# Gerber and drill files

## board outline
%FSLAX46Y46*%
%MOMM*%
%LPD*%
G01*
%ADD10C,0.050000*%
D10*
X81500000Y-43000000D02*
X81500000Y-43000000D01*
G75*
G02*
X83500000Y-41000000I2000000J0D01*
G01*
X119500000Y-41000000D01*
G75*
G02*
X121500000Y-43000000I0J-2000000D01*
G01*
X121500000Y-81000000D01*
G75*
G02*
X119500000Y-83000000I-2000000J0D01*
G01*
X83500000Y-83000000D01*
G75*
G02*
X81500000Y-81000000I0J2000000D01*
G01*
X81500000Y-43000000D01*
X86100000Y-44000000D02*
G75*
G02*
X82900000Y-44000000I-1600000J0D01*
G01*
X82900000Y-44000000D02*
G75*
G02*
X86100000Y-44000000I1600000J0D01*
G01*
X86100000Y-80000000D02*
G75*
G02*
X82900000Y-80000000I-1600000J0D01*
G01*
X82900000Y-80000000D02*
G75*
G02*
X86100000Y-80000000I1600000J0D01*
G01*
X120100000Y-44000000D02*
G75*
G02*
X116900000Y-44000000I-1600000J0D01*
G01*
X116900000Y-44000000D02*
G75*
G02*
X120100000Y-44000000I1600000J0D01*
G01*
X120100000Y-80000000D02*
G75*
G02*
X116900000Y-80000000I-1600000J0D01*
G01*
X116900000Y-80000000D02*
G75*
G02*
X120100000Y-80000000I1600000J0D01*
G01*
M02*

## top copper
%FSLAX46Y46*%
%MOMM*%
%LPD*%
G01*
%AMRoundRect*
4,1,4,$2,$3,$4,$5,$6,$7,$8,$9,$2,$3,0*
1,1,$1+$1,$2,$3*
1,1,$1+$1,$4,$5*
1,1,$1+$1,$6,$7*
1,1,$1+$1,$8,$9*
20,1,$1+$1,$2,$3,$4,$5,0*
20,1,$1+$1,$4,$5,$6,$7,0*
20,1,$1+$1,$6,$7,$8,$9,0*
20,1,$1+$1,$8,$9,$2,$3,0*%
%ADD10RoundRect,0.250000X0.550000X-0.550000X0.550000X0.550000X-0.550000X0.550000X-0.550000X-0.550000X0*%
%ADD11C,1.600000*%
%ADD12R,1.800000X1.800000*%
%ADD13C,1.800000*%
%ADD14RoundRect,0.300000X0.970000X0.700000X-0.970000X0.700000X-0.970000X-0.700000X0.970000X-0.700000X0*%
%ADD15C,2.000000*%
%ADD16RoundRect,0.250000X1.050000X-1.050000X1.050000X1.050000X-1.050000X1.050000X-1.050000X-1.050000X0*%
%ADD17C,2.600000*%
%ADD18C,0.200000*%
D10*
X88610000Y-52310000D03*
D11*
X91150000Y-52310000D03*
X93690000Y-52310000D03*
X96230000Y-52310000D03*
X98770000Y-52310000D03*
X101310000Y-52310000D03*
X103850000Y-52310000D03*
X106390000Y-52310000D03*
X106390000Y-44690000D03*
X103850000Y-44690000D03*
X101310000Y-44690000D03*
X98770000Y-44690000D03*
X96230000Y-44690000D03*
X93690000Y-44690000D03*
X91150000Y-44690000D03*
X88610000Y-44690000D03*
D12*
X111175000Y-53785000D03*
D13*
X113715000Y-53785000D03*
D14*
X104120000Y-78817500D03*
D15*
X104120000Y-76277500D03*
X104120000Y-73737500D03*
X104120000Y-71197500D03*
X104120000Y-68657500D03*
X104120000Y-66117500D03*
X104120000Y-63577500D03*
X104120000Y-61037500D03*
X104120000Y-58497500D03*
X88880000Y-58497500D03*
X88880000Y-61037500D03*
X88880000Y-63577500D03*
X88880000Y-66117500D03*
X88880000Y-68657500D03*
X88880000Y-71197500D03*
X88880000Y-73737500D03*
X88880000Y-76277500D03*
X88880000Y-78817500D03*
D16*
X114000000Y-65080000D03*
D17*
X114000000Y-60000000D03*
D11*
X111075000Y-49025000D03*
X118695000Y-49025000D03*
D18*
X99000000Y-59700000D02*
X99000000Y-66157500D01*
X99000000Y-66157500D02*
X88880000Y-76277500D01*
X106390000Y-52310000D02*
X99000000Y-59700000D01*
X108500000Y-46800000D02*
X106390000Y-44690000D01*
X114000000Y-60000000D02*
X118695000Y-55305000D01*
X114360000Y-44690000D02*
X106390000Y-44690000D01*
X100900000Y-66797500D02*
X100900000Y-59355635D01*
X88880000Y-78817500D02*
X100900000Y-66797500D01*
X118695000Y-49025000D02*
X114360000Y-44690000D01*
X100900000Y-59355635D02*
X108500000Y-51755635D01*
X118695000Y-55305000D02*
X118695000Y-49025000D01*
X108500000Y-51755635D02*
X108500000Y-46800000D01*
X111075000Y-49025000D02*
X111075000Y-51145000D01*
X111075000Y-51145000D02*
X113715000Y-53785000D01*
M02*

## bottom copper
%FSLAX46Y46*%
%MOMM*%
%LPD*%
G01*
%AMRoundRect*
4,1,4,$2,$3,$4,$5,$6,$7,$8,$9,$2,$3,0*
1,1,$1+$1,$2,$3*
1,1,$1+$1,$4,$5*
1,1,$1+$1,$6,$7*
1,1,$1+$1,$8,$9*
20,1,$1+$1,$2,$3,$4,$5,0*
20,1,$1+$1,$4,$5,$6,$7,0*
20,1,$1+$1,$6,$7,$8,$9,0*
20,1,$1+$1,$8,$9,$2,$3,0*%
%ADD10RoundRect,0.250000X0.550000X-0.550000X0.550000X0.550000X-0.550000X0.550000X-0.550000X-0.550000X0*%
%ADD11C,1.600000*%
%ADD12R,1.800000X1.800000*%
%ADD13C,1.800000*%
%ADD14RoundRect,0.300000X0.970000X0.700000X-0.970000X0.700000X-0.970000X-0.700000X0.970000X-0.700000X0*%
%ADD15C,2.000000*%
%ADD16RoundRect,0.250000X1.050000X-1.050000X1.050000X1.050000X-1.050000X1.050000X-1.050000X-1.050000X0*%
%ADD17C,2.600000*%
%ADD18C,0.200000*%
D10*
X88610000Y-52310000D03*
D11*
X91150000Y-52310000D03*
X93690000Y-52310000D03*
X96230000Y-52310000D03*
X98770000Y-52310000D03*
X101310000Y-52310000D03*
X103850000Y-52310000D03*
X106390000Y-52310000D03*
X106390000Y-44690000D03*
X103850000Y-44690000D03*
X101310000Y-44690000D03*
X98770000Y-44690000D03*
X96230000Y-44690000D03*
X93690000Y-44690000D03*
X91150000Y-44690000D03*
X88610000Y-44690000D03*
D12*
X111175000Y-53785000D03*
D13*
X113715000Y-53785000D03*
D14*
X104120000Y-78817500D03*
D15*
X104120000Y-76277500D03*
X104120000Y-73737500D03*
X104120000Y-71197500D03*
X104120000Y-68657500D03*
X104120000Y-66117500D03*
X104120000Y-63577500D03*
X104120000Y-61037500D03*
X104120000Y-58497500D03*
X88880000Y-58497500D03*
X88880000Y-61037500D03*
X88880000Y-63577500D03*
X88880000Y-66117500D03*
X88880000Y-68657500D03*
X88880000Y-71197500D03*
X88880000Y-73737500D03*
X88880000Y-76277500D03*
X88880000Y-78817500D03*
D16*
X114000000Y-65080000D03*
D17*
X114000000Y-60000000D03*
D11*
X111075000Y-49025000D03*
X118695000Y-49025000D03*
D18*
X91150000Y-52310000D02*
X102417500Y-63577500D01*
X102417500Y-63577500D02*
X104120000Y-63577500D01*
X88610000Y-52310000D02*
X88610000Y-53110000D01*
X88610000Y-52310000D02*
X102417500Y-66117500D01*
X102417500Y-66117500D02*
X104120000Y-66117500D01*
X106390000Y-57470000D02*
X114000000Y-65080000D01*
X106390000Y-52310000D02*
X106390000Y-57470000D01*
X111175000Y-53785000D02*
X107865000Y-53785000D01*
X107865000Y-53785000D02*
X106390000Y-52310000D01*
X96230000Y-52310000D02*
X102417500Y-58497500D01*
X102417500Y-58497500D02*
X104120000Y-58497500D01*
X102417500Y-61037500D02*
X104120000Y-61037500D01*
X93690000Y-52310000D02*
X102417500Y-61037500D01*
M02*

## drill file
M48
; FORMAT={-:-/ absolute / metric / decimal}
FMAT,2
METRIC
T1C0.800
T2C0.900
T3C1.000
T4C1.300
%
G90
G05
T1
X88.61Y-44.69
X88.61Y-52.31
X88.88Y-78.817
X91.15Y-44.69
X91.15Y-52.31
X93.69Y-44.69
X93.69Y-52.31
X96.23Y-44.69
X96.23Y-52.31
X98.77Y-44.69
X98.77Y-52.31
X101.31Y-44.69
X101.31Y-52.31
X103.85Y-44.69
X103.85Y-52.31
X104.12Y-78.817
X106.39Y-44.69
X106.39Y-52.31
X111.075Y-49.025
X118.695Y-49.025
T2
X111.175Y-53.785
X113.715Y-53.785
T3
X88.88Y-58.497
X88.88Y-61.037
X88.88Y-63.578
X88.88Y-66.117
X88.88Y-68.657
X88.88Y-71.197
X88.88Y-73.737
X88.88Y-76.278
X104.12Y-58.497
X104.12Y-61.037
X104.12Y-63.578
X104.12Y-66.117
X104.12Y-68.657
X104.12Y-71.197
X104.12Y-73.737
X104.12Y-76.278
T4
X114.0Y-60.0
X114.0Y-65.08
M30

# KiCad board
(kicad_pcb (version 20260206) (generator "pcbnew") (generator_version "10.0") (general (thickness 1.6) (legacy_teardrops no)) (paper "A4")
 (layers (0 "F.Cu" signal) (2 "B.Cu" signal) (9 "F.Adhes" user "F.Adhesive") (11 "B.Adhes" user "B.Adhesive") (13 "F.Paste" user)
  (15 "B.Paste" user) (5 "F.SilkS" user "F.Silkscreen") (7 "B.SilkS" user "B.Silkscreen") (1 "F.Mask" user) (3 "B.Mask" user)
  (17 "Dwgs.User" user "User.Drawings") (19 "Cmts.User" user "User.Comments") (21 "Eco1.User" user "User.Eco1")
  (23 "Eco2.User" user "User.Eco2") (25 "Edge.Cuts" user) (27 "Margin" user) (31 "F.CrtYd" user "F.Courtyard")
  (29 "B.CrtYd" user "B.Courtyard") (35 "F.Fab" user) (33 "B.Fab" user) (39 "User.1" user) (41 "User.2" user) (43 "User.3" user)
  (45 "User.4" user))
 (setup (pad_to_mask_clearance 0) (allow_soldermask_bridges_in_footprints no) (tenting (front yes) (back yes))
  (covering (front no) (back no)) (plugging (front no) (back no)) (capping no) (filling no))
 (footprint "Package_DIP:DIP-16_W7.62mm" (layer "F.Cu") (at 88.61 52.31 90)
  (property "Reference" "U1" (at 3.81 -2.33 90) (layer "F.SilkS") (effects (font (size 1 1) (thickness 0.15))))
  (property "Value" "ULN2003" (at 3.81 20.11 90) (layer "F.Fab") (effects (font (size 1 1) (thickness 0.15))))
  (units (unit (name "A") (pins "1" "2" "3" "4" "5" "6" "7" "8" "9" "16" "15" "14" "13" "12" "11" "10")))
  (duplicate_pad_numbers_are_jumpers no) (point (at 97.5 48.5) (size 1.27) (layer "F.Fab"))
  (pad "1" thru_hole roundrect (at 0 0 90) (size 1.6 1.6) (drill 0.8) (layers "*.Cu" "*.Mask") (remove_unused_layers no)
   (roundrect_rratio 0.15625) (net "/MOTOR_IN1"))
  (pad "2" thru_hole circle (at 0 2.54 90) (size 1.6 1.6) (drill 0.8) (layers "*.Cu" "*.Mask") (remove_unused_layers no) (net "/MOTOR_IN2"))
  (pad "3" thru_hole circle (at 0 5.08 90) (size 1.6 1.6) (drill 0.8) (layers "*.Cu" "*.Mask") (remove_unused_layers no) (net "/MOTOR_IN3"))
  (pad "4" thru_hole circle (at 0 7.62 90) (size 1.6 1.6) (drill 0.8) (layers "*.Cu" "*.Mask") (remove_unused_layers no) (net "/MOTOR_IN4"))
  (pad "5" thru_hole circle (at 0 10.16 90) (size 1.6 1.6) (drill 0.8) (layers "*.Cu" "*.Mask") (remove_unused_layers no)
   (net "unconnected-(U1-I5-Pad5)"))
  (pad "6" thru_hole circle (at 0 12.7 90) (size 1.6 1.6) (drill 0.8) (layers "*.Cu" "*.Mask") (remove_unused_layers no)
   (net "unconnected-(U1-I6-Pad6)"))
  (pad "7" thru_hole circle (at 0 15.24 90) (size 1.6 1.6) (drill 0.8) (layers "*.Cu" "*.Mask") (remove_unused_layers no)
   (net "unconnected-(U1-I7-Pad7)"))
  (pad "8" thru_hole circle (at 0 17.78 90) (size 1.6 1.6) (drill 0.8) (layers "*.Cu" "*.Mask") (remove_unused_layers no) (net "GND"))
  (pad "9" thru_hole circle (at 7.62 17.78 90) (size 1.6 1.6) (drill 0.8) (layers "*.Cu" "*.Mask") (remove_unused_layers no) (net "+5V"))
  (pad "10" thru_hole circle (at 7.62 15.24 90) (size 1.6 1.6) (drill 0.8) (layers "*.Cu" "*.Mask") (remove_unused_layers no)
   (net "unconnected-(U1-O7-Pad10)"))
  (pad "11" thru_hole circle (at 7.62 12.7 90) (size 1.6 1.6) (drill 0.8) (layers "*.Cu" "*.Mask") (remove_unused_layers no)
   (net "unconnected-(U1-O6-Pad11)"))
  (pad "12" thru_hole circle (at 7.62 10.16 90) (size 1.6 1.6) (drill 0.8) (layers "*.Cu" "*.Mask") (remove_unused_layers no)
   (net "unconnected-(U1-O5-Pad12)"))
  (pad "13" thru_hole circle (at 7.62 7.62 90) (size 1.6 1.6) (drill 0.8) (layers "*.Cu" "*.Mask") (remove_unused_layers no)
   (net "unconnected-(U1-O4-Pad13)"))
  (pad "14" thru_hole circle (at 7.62 5.08 90) (size 1.6 1.6) (drill 0.8) (layers "*.Cu" "*.Mask") (remove_unused_layers no)
   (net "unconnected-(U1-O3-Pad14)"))
  (pad "15" thru_hole circle (at 7.62 2.54 90) (size 1.6 1.6) (drill 0.8) (layers "*.Cu" "*.Mask") (remove_unused_layers no)
   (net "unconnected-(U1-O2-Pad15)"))
  (pad "16" thru_hole circle (at 7.62 0 90) (size 1.6 1.6) (drill 0.8) (layers "*.Cu" "*.Mask") (remove_unused_layers no)
   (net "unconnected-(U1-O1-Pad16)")))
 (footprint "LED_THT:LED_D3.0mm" (layer "F.Cu") (at 111.175 53.785)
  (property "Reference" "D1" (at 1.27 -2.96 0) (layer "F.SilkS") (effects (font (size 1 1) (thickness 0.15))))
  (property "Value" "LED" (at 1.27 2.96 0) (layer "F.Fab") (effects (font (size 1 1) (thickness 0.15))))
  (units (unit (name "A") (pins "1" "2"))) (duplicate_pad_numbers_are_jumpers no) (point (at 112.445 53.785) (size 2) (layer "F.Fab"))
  (pad "1" thru_hole rect (at 0 0) (size 1.8 1.8) (drill 0.9) (layers "*.Cu" "*.Mask") (remove_unused_layers no) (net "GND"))
  (pad "2" thru_hole circle (at 2.54 0) (size 1.8 1.8) (drill 0.9) (layers "*.Cu" "*.Mask") (remove_unused_layers no) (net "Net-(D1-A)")))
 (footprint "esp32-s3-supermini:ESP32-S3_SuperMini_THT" (layer "F.Cu") (at 104.12 78.8175 180)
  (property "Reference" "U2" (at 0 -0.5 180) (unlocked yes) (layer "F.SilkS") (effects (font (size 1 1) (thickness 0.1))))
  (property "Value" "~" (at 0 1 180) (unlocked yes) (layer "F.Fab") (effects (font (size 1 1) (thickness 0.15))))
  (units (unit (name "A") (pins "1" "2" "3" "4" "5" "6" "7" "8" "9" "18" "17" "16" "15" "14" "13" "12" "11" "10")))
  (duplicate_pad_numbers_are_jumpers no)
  (pad "1" thru_hole roundrect (at 0 0 180) (size 2.54 2) (drill 0.8) (layers "*.Cu" "*.Mask") (remove_unused_layers no)
   (roundrect_rratio 0.15) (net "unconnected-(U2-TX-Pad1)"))
  (pad "2" thru_hole circle (at 0 2.54 180) (size 2 2) (drill 1) (layers "*.Cu" "*.Mask") (remove_unused_layers no)
   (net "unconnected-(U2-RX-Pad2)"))
  (pad "3" thru_hole circle (at 0 5.08 180) (size 2 2) (drill 1) (layers "*.Cu" "*.Mask") (remove_unused_layers no)
   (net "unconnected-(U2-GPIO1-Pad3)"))
  (pad "4" thru_hole circle (at 0 7.62 180) (size 2 2) (drill 1) (layers "*.Cu" "*.Mask") (remove_unused_layers no)
   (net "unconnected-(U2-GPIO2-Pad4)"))
  (pad "5" thru_hole circle (at 0 10.16 180) (size 2 2) (drill 1) (layers "*.Cu" "*.Mask") (remove_unused_layers no)
   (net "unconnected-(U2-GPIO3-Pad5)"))
  (pad "6" thru_hole circle (at 0 12.7 180) (size 2 2) (drill 1) (layers "*.Cu" "*.Mask") (remove_unused_layers no) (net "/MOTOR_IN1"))
  (pad "7" thru_hole circle (at 0 15.24 180) (size 2 2) (drill 1) (layers "*.Cu" "*.Mask") (remove_unused_layers no) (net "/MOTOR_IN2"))
  (pad "8" thru_hole circle (at 0 17.78 180) (size 2 2) (drill 1) (layers "*.Cu" "*.Mask") (remove_unused_layers no) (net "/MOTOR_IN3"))
  (pad "9" thru_hole circle (at 0 20.32 180) (size 2 2) (drill 1) (layers "*.Cu" "*.Mask") (remove_unused_layers no) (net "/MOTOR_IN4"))
  (pad "10" thru_hole circle (at 15.24 20.32 180) (size 2 2) (drill 1) (layers "*.Cu" "*.Mask") (remove_unused_layers no)
   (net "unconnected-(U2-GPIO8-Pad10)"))
  (pad "11" thru_hole circle (at 15.24 17.78 180) (size 2 2) (drill 1) (layers "*.Cu" "*.Mask") (remove_unused_layers no)
   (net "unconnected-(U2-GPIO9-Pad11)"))
  (pad "12" thru_hole circle (at 15.24 15.24 180) (size 2 2) (drill 1) (layers "*.Cu" "*.Mask") (remove_unused_layers no)
   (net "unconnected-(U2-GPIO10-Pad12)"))
  (pad "13" thru_hole circle (at 15.24 12.7 180) (size 2 2) (drill 1) (layers "*.Cu" "*.Mask") (remove_unused_layers no)
   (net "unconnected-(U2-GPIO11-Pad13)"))
  (pad "14" thru_hole circle (at 15.24 10.16 180) (size 2 2) (drill 1) (layers "*.Cu" "*.Mask") (remove_unused_layers no)
   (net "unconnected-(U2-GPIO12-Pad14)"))
  (pad "15" thru_hole circle (at 15.24 7.62 180) (size 2 2) (drill 1) (layers "*.Cu" "*.Mask") (remove_unused_layers no)
   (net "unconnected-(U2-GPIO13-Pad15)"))
  (pad "16" thru_hole circle (at 15.24 5.08 180) (size 2 2) (drill 1) (layers "*.Cu" "*.Mask") (remove_unused_layers no)
   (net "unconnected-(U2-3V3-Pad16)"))
  (pad "17" thru_hole circle (at 15.24 2.54 180) (size 2 2) (drill 1) (layers "*.Cu" "*.Mask") (remove_unused_layers no) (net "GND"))
  (pad "18" thru_hole circle (at 15.24 0 180) (size 2 2) (drill 0.8) (layers "*.Cu" "*.Mask") (remove_unused_layers no) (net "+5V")))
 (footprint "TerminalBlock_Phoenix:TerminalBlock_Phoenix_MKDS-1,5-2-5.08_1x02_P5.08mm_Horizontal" (layer "F.Cu") (at 114 65.08 90)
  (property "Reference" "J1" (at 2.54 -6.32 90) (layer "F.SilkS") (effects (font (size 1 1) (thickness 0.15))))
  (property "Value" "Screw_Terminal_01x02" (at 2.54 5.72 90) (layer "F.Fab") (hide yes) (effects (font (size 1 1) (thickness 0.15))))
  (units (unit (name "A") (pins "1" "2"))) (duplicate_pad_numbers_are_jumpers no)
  (pad "1" thru_hole roundrect (at 0 0 90) (size 2.6 2.6) (drill 1.3) (layers "*.Cu" "*.Mask") (remove_unused_layers no)
   (roundrect_rratio 0.096154) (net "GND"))
  (pad "2" thru_hole circle (at 5.08 0 90) (size 2.6 2.6) (drill 1.3) (layers "*.Cu" "*.Mask") (remove_unused_layers no) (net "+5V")))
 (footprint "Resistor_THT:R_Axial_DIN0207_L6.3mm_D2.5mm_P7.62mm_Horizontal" (layer "F.Cu") (at 111.075 49.025)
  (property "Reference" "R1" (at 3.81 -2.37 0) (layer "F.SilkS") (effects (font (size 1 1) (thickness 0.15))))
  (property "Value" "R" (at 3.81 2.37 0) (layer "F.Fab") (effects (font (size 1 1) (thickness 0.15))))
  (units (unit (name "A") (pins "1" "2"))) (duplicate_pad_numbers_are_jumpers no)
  (pad "1" thru_hole circle (at 0 0) (size 1.6 1.6) (drill 0.8) (layers "*.Cu" "*.Mask") (remove_unused_layers no) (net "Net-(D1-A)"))
  (pad "2" thru_hole circle (at 7.62 0) (size 1.6 1.6) (drill 0.8) (layers "*.Cu" "*.Mask") (remove_unused_layers no) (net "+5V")))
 (gr_rect (start 81.5 41) (end 121.5 83) (radius 2) (stroke (width 0.05) (type solid)) (fill no) (layer "Edge.Cuts"))
 (gr_circle (center 84.5 44) (end 86.1 44) (stroke (width 0.05) (type solid)) (fill no) (layer "Edge.Cuts"))
 (gr_circle (center 84.5 80) (end 86.1 80) (stroke (width 0.05) (type solid)) (fill no) (layer "Edge.Cuts"))
 (gr_circle (center 118.5 44) (end 120.1 44) (stroke (width 0.05) (type solid)) (fill no) (layer "Edge.Cuts"))
 (gr_circle (center 118.5 80) (end 120.1 80) (stroke (width 0.05) (type solid)) (fill no) (layer "Edge.Cuts"))
 (segment (start 91.15 52.31) (end 102.4175 63.5775) (width 0.2) (layer "B.Cu") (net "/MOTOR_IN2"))
 (segment (start 102.4175 63.5775) (end 104.12 63.5775) (width 0.2) (layer "B.Cu") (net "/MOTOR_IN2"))
 (segment (start 88.61 52.31) (end 88.61 53.11) (width 0.2) (layer "B.Cu") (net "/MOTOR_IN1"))
 (segment (start 88.61 52.31) (end 102.4175 66.1175) (width 0.2) (layer "B.Cu") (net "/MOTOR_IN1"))
 (segment (start 102.4175 66.1175) (end 104.12 66.1175) (width 0.2) (layer "B.Cu") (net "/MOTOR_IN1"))
 (segment (start 99 59.7) (end 99 66.1575) (width 0.2) (layer "F.Cu") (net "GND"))
 (segment (start 99 66.1575) (end 88.88 76.2775) (width 0.2) (layer "F.Cu") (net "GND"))
 (segment (start 106.39 52.31) (end 99 59.7) (width 0.2) (layer "F.Cu") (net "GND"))
 (segment (start 106.39 57.47) (end 114 65.08) (width 0.2) (layer "B.Cu") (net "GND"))
 (segment (start 106.39 52.31) (end 106.39 57.47) (width 0.2) (layer "B.Cu") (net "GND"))
 (segment (start 111.175 53.785) (end 107.865 53.785) (width 0.2) (layer "B.Cu") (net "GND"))
 (segment (start 107.865 53.785) (end 106.39 52.31) (width 0.2) (layer "B.Cu") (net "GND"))
 (segment (start 108.5 46.8) (end 106.39 44.69) (width 0.2) (layer "F.Cu") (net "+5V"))
 (segment (start 114 60) (end 118.695 55.305) (width 0.2) (layer "F.Cu") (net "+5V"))
 (segment (start 114.36 44.69) (end 106.39 44.69) (width 0.2) (layer "F.Cu") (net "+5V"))
 (segment (start 100.9 66.7975) (end 100.9 59.355635) (width 0.2) (layer "F.Cu") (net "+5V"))
 (segment (start 88.88 78.8175) (end 100.9 66.7975) (width 0.2) (layer "F.Cu") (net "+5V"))
 (segment (start 118.695 49.025) (end 114.36 44.69) (width 0.2) (layer "F.Cu") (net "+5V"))
 (segment (start 100.9 59.355635) (end 108.5 51.755635) (width 0.2) (layer "F.Cu") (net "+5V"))
 (segment (start 118.695 55.305) (end 118.695 49.025) (width 0.2) (layer "F.Cu") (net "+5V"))
 (segment (start 108.5 51.755635) (end 108.5 46.8) (width 0.2) (layer "F.Cu") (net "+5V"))
 (segment (start 96.23 52.31) (end 102.4175 58.4975) (width 0.2) (layer "B.Cu") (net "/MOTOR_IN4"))
 (segment (start 102.4175 58.4975) (end 104.12 58.4975) (width 0.2) (layer "B.Cu") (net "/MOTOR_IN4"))
 (segment (start 102.4175 61.0375) (end 104.12 61.0375) (width 0.2) (layer "B.Cu") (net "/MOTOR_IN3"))
 (segment (start 93.69 52.31) (end 102.4175 61.0375) (width 0.2) (layer "B.Cu") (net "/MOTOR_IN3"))
 (segment (start 111.075 49.025) (end 111.075 51.145) (width 0.2) (layer "F.Cu") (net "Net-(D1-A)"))
 (segment (start 111.075 51.145) (end 113.715 53.785) (width 0.2) (layer "F.Cu") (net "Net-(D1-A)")))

